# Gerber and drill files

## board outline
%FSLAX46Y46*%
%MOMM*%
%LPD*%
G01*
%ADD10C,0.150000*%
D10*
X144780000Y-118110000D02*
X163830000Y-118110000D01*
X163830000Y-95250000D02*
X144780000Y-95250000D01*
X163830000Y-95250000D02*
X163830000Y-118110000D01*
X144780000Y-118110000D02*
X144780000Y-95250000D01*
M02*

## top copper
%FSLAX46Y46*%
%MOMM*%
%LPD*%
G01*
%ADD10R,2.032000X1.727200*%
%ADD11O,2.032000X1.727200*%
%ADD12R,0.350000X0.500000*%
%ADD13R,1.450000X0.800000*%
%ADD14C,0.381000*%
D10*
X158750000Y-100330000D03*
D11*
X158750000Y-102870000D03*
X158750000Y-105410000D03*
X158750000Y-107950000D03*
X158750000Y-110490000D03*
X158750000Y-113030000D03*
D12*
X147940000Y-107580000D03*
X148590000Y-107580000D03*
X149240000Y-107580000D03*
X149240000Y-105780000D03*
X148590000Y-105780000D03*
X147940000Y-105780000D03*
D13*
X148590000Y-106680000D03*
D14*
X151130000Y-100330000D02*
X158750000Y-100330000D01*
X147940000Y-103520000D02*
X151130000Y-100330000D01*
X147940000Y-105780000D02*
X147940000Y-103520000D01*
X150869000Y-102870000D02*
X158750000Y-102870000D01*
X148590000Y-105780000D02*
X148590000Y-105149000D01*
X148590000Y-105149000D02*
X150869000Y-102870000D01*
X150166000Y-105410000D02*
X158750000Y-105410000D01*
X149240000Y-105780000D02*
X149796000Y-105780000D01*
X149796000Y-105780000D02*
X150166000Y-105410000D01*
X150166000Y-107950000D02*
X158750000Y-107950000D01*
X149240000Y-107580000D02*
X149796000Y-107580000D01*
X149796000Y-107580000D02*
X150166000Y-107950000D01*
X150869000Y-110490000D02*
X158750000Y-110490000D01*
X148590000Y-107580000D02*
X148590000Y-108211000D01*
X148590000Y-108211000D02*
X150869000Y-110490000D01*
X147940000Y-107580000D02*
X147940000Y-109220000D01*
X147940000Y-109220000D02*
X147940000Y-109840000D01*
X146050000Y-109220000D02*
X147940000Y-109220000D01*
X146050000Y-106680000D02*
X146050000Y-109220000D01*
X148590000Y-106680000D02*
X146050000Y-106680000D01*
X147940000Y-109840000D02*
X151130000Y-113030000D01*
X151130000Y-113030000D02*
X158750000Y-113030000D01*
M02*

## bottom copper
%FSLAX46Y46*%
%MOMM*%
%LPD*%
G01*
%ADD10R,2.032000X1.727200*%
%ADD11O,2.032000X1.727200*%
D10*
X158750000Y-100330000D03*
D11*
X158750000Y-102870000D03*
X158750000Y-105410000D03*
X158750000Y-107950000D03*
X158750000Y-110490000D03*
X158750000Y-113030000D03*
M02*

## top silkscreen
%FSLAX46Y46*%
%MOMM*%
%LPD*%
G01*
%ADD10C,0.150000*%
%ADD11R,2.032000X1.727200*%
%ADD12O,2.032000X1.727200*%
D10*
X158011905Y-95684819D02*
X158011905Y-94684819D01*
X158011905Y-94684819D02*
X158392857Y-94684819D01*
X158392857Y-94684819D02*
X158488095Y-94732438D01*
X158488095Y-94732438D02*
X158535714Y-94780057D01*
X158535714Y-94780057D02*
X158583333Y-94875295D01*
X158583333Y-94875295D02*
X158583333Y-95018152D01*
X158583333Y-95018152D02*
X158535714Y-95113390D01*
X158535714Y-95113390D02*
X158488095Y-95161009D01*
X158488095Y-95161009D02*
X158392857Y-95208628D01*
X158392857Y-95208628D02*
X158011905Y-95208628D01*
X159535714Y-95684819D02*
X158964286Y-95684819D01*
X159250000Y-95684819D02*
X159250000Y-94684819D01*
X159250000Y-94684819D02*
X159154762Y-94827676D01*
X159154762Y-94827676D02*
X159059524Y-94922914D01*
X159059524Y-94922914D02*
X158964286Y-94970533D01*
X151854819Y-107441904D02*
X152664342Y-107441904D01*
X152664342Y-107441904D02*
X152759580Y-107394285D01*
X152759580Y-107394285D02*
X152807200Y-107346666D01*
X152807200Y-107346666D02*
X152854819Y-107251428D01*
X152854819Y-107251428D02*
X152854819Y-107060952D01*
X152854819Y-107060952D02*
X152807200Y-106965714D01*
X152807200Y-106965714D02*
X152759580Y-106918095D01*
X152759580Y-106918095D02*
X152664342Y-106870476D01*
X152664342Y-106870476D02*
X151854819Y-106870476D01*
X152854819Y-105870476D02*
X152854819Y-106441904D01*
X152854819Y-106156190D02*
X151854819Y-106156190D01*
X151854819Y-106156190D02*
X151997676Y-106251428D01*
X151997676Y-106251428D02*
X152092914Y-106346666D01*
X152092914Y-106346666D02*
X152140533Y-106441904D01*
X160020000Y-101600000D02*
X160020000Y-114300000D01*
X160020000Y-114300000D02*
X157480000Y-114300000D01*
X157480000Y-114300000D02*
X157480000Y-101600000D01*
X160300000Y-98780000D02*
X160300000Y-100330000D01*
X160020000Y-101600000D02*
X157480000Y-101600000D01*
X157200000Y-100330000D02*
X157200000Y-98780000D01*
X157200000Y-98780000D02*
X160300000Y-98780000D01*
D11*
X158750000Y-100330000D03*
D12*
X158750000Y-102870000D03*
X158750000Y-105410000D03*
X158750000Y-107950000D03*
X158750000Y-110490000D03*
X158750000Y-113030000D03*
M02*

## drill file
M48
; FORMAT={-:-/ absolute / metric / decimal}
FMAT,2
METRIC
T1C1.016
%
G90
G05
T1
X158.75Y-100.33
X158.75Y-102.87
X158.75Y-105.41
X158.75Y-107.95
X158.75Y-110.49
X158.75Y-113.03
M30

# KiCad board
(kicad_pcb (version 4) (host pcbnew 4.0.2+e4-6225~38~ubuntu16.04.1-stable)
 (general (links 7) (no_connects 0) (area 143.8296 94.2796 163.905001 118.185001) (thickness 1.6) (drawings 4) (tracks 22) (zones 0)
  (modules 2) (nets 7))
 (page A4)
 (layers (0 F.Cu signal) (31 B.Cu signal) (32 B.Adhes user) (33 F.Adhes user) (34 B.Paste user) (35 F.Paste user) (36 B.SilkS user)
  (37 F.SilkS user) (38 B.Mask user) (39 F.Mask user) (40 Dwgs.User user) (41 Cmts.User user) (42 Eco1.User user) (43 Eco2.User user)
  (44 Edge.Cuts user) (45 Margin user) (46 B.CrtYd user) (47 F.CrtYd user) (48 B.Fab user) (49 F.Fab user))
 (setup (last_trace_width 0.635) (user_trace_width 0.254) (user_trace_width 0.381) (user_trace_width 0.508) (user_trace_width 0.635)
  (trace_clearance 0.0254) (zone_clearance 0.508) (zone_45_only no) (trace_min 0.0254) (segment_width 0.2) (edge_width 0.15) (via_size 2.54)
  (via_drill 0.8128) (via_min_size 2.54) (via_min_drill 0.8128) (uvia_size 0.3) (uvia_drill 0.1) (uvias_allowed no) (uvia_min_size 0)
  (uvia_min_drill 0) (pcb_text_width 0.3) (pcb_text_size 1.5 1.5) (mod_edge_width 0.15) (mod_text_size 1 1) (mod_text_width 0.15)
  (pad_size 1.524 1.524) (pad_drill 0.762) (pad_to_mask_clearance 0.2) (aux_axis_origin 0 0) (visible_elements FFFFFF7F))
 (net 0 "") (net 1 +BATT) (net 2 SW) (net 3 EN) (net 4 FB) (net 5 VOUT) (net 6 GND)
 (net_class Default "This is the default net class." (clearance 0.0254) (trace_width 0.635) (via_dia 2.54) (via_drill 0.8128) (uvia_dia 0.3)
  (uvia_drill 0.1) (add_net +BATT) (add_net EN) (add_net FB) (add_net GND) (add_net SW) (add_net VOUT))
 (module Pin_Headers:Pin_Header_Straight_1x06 (layer F.Cu) (at 158.75 100.33)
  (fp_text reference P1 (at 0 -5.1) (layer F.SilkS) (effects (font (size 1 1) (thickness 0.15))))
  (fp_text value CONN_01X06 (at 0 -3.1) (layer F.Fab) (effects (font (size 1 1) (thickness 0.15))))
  (fp_line (start 1.27 1.27) (end 1.27 13.97) (layer F.SilkS) (width 0.15))
  (fp_line (start 1.27 13.97) (end -1.27 13.97) (layer F.SilkS) (width 0.15))
  (fp_line (start -1.27 13.97) (end -1.27 1.27) (layer F.SilkS) (width 0.15))
  (fp_line (start 1.55 -1.55) (end 1.55 0) (layer F.SilkS) (width 0.15))
  (fp_line (start 1.27 1.27) (end -1.27 1.27) (layer F.SilkS) (width 0.15))
  (fp_line (start -1.55 0) (end -1.55 -1.55) (layer F.SilkS) (width 0.15))
  (fp_line (start -1.55 -1.55) (end 1.55 -1.55) (layer F.SilkS) (width 0.15))
  (pad 1 thru_hole rect (at 0 0) (size 2.032 1.7272) (drill 1.016) (layers *.Cu *.Mask F.SilkS) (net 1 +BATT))
  (pad 2 thru_hole oval (at 0 2.54) (size 2.032 1.7272) (drill 1.016) (layers *.Cu *.Mask F.SilkS) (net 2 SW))
  (pad 3 thru_hole oval (at 0 5.08) (size 2.032 1.7272) (drill 1.016) (layers *.Cu *.Mask F.SilkS) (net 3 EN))
  (pad 4 thru_hole oval (at 0 7.62) (size 2.032 1.7272) (drill 1.016) (layers *.Cu *.Mask F.SilkS) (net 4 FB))
  (pad 5 thru_hole oval (at 0 10.16) (size 2.032 1.7272) (drill 1.016) (layers *.Cu *.Mask F.SilkS) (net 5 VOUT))
  (pad 6 thru_hole oval (at 0 12.7) (size 2.032 1.7272) (drill 1.016) (layers *.Cu *.Mask F.SilkS) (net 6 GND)))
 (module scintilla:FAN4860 (layer F.Cu) (at 148.59 106.68 90)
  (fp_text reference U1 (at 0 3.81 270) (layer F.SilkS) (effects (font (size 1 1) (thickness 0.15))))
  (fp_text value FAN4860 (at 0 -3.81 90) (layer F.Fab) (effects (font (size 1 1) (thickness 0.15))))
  (pad 1 smd rect (at -0.9 -0.65 90) (size 0.5 0.35) (layers F.Cu F.Paste F.Mask) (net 6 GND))
  (pad 2 smd rect (at -0.9 0 90) (size 0.5 0.35) (layers F.Cu F.Paste F.Mask) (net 5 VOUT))
  (pad 3 smd rect (at -0.9 0.65 90) (size 0.5 0.35) (layers F.Cu F.Paste F.Mask) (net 4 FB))
  (pad 4 smd rect (at 0.9 0.65 90) (size 0.5 0.35) (layers F.Cu F.Paste F.Mask) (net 3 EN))
  (pad 5 smd rect (at 0.9 0 90) (size 0.5 0.35) (layers F.Cu F.Paste F.Mask) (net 2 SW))
  (pad 6 smd rect (at 0.9 -0.65 90) (size 0.5 0.35) (layers F.Cu F.Paste F.Mask) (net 1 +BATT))
  (pad 7 smd rect (at 0 0 90) (size 0.8 1.45) (layers F.Cu F.Paste F.Mask) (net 6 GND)))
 (gr_line (start 144.78 118.11) (end 163.83 118.11) (layer Edge.Cuts) (width 0.15))
 (gr_line (start 163.83 95.25) (end 144.78 95.25) (layer Edge.Cuts) (width 0.15))
 (gr_line (start 163.83 95.25) (end 163.83 118.11) (layer Edge.Cuts) (width 0.15))
 (gr_line (start 144.78 118.11) (end 144.78 95.25) (layer Edge.Cuts) (width 0.15))
 (segment (start 151.13 100.33) (end 158.75 100.33) (width 0.381) (layer F.Cu) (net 1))
 (segment (start 147.94 103.52) (end 151.13 100.33) (width 0.381) (layer F.Cu) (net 1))
 (segment (start 147.94 105.78) (end 147.94 103.52) (width 0.381) (layer F.Cu) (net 1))
 (segment (start 150.869 102.87) (end 158.75 102.87) (width 0.381) (layer F.Cu) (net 2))
 (segment (start 148.59 105.78) (end 148.59 105.149) (width 0.381) (layer F.Cu) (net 2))
 (segment (start 148.59 105.149) (end 150.869 102.87) (width 0.381) (layer F.Cu) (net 2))
 (segment (start 150.166 105.41) (end 158.75 105.41) (width 0.381) (layer F.Cu) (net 3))
 (segment (start 149.24 105.78) (end 149.796 105.78) (width 0.381) (layer F.Cu) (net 3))
 (segment (start 149.796 105.78) (end 150.166 105.41) (width 0.381) (layer F.Cu) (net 3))
 (segment (start 150.166 107.95) (end 158.75 107.95) (width 0.381) (layer F.Cu) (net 4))
 (segment (start 149.24 107.58) (end 149.796 107.58) (width 0.381) (layer F.Cu) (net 4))
 (segment (start 149.796 107.58) (end 150.166 107.95) (width 0.381) (layer F.Cu) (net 4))
 (segment (start 150.869 110.49) (end 158.75 110.49) (width 0.381) (layer F.Cu) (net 5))
 (segment (start 148.59 107.58) (end 148.59 108.211) (width 0.381) (layer F.Cu) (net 5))
 (segment (start 148.59 108.211) (end 150.869 110.49) (width 0.381) (layer F.Cu) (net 5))
 (segment (start 147.94 107.58) (end 147.94 109.22) (width 0.381) (layer F.Cu) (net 6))
 (segment (start 147.94 109.22) (end 147.94 109.84) (width 0.381) (layer F.Cu) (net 6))
 (segment (start 146.05 109.22) (end 147.94 109.22) (width 0.381) (layer F.Cu) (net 6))
 (segment (start 146.05 106.68) (end 146.05 109.22) (width 0.381) (layer F.Cu) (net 6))
 (segment (start 148.59 106.68) (end 146.05 106.68) (width 0.381) (layer F.Cu) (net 6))
 (segment (start 147.94 109.84) (end 151.13 113.03) (width 0.381) (layer F.Cu) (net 6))
 (segment (start 151.13 113.03) (end 158.75 113.03) (width 0.381) (layer F.Cu) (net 6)))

